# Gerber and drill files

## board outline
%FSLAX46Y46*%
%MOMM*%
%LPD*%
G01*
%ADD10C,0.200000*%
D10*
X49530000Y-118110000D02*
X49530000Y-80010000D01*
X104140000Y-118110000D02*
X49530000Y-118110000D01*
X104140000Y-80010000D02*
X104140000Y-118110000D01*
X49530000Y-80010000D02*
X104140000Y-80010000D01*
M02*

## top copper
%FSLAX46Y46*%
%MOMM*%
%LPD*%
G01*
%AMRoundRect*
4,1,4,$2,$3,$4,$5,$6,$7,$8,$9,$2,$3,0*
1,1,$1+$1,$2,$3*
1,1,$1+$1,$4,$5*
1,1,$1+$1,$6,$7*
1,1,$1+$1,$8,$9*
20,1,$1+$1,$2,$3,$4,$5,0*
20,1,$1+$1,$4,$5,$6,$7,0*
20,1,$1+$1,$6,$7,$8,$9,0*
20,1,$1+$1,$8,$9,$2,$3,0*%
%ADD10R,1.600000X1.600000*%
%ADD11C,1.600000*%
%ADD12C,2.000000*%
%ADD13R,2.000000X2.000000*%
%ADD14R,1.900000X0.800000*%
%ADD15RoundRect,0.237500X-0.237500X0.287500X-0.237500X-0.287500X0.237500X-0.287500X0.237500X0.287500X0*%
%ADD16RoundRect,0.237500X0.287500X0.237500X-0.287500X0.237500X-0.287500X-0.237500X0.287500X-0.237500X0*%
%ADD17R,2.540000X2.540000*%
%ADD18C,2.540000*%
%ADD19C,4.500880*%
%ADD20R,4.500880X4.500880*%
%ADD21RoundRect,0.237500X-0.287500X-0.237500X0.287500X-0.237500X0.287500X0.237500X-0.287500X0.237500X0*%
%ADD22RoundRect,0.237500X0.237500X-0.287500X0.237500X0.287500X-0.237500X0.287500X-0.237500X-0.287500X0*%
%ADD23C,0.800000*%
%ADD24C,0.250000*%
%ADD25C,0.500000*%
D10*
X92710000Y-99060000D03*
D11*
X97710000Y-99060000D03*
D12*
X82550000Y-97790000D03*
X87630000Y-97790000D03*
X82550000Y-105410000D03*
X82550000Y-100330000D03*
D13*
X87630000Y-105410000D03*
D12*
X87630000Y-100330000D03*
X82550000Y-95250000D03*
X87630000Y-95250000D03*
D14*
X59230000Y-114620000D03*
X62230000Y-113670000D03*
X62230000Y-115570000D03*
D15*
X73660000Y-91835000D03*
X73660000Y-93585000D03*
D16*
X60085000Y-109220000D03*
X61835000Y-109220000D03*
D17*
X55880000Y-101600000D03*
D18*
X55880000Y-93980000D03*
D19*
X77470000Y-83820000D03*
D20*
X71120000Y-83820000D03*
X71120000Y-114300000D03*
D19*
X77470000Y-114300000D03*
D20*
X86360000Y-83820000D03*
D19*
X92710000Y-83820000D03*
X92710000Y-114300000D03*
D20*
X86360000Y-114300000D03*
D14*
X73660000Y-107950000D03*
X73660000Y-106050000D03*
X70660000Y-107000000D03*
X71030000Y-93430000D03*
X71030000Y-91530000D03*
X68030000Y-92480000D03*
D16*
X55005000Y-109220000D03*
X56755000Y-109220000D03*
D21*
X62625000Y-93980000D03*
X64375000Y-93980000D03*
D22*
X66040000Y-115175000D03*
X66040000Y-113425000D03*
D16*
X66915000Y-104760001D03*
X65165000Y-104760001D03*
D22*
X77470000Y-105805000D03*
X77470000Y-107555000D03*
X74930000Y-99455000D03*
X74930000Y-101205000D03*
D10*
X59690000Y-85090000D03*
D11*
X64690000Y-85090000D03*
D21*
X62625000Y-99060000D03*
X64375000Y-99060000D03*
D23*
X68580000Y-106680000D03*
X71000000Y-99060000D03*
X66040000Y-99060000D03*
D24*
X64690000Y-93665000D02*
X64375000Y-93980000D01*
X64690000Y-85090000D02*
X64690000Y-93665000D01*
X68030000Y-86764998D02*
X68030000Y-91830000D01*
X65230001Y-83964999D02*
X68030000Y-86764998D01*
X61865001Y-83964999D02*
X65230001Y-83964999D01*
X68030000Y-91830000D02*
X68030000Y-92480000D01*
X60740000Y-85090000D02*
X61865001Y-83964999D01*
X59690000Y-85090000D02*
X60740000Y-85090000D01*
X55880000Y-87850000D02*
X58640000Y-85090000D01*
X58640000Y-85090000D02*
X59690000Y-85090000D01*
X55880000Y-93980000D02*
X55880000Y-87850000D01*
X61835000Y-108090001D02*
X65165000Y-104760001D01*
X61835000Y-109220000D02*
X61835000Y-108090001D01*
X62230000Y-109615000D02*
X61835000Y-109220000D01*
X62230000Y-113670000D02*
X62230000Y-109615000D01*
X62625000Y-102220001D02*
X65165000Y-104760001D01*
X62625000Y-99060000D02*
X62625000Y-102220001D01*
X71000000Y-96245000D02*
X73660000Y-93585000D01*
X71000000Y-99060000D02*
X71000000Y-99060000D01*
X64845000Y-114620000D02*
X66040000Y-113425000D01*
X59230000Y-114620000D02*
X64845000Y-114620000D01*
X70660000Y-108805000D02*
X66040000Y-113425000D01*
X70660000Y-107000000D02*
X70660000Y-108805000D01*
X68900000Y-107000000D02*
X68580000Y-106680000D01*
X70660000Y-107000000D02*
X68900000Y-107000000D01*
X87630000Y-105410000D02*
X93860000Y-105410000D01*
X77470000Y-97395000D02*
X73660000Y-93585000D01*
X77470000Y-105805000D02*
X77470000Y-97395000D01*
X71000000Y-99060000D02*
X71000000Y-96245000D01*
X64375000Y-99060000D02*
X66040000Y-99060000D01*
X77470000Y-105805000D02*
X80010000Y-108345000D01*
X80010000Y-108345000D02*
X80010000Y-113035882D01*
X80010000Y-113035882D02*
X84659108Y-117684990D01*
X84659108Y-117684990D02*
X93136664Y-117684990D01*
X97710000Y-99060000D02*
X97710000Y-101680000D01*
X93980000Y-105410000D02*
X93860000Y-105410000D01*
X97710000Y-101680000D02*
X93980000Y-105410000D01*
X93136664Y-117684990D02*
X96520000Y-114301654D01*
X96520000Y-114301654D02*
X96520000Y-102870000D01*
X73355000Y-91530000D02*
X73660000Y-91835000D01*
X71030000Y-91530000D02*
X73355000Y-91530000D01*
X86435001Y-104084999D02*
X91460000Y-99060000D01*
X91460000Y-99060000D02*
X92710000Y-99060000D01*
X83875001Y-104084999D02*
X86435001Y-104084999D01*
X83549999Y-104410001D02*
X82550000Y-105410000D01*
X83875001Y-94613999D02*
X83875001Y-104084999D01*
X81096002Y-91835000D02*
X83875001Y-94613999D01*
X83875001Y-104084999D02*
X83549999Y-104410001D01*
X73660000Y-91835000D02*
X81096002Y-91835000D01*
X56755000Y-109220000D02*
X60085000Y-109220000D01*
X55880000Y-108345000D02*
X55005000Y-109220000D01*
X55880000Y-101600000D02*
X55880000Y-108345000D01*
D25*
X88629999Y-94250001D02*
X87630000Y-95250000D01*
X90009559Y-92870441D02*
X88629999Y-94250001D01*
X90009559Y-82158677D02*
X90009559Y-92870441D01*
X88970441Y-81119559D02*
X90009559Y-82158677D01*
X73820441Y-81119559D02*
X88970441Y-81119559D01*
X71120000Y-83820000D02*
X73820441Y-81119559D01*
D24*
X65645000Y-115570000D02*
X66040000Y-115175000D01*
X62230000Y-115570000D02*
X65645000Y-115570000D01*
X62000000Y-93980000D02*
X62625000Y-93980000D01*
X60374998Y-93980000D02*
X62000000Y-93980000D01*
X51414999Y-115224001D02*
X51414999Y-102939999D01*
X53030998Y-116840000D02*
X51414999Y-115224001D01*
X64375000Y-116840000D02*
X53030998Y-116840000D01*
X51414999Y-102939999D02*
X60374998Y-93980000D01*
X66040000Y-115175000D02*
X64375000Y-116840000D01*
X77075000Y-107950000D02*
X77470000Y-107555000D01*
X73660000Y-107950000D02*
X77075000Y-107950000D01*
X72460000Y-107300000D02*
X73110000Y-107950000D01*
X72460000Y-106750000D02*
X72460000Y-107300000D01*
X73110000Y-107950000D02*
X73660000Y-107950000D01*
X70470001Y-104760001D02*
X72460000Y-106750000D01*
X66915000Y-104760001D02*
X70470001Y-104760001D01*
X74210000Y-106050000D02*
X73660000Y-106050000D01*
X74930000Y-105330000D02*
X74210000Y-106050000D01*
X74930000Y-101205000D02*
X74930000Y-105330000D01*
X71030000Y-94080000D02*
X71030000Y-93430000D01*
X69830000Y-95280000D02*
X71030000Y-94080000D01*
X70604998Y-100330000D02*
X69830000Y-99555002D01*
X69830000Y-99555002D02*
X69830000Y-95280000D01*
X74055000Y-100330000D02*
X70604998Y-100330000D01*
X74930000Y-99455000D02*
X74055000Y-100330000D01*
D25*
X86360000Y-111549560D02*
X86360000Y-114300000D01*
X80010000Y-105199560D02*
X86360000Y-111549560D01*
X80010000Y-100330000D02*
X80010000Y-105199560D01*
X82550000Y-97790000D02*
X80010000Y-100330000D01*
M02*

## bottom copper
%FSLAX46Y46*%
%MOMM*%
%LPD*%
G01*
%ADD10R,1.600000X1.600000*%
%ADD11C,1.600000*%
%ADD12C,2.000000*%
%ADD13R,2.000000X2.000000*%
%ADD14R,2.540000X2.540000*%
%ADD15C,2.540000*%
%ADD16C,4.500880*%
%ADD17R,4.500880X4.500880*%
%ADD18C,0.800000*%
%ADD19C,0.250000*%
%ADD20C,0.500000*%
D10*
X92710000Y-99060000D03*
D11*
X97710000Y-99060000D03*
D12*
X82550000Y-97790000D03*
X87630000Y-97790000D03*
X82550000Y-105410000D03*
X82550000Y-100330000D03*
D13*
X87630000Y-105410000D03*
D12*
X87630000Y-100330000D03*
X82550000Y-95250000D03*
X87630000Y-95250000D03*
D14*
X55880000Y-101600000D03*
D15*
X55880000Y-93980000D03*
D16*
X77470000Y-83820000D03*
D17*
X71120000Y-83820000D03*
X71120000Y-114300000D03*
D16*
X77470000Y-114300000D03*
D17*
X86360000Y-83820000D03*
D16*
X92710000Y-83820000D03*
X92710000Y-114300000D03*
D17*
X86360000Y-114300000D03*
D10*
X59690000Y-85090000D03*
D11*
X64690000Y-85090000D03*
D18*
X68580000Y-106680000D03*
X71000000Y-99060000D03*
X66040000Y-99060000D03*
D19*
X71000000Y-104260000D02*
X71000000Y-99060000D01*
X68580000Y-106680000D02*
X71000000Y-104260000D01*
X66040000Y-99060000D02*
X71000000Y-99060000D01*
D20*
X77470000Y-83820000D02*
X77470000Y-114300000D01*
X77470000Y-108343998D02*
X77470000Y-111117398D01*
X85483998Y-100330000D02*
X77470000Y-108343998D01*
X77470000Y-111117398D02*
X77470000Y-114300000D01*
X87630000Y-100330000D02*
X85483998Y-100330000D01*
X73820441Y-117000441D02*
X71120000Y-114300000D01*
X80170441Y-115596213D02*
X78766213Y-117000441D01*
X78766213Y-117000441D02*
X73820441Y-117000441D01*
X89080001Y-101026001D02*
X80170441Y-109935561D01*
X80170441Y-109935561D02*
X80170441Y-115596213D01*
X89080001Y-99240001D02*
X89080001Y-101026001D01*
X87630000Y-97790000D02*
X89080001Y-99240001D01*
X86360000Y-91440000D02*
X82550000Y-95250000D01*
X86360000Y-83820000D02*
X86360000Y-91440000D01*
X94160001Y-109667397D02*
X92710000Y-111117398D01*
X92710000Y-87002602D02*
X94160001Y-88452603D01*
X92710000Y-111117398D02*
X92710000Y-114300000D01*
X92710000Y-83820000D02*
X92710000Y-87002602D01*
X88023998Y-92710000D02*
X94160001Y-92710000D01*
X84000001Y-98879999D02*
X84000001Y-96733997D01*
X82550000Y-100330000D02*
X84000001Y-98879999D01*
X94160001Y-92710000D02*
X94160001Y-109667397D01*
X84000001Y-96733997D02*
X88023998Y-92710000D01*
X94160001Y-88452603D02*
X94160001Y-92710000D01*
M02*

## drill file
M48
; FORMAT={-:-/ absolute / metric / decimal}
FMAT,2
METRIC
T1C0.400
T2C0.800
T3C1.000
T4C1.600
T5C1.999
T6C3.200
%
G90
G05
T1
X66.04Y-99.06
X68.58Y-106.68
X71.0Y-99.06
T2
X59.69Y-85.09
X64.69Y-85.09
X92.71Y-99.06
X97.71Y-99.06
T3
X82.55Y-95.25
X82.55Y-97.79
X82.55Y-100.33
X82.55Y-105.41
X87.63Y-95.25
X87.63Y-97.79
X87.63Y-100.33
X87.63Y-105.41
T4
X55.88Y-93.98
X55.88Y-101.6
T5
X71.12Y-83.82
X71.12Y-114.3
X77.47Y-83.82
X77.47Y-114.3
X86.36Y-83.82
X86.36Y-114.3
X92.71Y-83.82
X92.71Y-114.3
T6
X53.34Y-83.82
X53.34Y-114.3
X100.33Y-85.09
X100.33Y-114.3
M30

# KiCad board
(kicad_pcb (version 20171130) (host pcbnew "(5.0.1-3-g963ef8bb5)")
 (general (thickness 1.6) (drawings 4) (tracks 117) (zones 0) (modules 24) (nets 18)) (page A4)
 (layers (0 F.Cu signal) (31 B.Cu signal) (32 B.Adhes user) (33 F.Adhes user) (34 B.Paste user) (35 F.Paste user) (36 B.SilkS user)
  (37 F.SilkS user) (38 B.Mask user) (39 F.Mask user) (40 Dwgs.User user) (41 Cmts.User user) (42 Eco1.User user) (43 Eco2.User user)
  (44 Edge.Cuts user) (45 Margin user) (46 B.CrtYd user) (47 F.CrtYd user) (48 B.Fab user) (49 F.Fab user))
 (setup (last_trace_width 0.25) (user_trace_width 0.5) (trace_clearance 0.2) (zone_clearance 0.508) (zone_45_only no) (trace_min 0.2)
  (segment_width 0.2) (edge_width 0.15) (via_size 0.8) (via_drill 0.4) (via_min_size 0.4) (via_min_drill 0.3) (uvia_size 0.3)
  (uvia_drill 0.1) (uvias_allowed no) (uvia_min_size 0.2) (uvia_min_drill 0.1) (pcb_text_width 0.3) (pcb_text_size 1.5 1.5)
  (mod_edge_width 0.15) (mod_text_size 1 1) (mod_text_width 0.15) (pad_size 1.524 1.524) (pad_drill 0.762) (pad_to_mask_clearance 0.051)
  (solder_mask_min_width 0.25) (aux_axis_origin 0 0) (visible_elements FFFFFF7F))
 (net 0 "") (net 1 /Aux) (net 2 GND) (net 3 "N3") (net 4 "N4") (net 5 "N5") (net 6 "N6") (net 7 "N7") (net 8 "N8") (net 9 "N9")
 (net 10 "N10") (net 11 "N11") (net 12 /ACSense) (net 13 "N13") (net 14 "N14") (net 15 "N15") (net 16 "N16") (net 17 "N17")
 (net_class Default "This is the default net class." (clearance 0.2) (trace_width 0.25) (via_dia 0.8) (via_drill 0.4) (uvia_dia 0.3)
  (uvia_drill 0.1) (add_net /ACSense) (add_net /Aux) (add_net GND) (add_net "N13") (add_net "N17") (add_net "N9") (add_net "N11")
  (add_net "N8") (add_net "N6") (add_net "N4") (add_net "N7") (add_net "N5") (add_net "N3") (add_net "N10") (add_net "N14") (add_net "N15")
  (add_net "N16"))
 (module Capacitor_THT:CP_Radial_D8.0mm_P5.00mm (layer F.Cu) (at 92.71 99.06)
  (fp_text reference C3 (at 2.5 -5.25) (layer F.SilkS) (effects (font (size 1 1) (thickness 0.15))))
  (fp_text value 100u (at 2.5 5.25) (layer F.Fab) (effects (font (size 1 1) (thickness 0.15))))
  (pad 1 thru_hole rect (at 0 0) (size 1.6 1.6) (drill 0.8) (layers *.Cu *.Mask) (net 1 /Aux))
  (pad 2 thru_hole circle (at 5 0) (size 1.6 1.6) (drill 0.8) (layers *.Cu *.Mask) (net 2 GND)))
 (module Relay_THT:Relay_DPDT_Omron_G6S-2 (layer F.Cu) (at 87.63 105.41 180)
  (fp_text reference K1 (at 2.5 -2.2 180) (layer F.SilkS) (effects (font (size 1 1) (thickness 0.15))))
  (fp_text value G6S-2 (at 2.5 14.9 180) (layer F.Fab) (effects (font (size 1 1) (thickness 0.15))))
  (pad 7 thru_hole circle (at 5.08 7.62 90) (size 2 2) (drill 1) (layers *.Cu *.Mask) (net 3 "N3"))
  (pad 4 thru_hole circle (at 0 7.62 90) (size 2 2) (drill 1) (layers *.Cu *.Mask) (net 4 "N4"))
  (pad 10 thru_hole circle (at 5.08 0 180) (size 2 2) (drill 1) (layers *.Cu *.Mask) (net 1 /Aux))
  (pad 8 thru_hole circle (at 5.08 5.08 180) (size 2 2) (drill 1) (layers *.Cu *.Mask) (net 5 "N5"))
  (pad 1 thru_hole rect (at 0 0 180) (size 2 2) (drill 1) (layers *.Cu *.Mask) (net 2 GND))
  (pad 3 thru_hole circle (at 0 5.08 180) (size 2 2) (drill 1) (layers *.Cu *.Mask) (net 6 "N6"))
  (pad 6 thru_hole circle (at 5.08 10.16 180) (size 2 2) (drill 1) (layers *.Cu *.Mask) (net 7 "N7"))
  (pad 5 thru_hole circle (at 0 10.16 180) (size 2 2) (drill 1) (layers *.Cu *.Mask) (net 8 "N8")))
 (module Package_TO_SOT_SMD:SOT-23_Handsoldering (layer F.Cu) (at 60.73 114.62 180)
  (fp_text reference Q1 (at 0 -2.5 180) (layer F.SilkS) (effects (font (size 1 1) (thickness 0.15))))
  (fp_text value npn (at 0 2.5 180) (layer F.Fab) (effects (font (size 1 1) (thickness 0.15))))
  (pad 3 smd rect (at 1.5 0 180) (size 1.9 0.8) (layers F.Cu F.Paste F.Mask) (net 2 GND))
  (pad 2 smd rect (at -1.5 0.95 180) (size 1.9 0.8) (layers F.Cu F.Paste F.Mask) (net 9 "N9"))
  (pad 1 smd rect (at -1.5 -0.95 180) (size 1.9 0.8) (layers F.Cu F.Paste F.Mask) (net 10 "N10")))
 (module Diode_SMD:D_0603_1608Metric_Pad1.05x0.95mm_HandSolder (layer F.Cu) (at 73.66 92.71 270)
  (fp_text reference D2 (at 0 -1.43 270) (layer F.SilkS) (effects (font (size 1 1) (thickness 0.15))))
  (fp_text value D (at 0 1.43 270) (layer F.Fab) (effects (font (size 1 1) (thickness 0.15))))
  (pad 1 smd roundrect (at -0.875 0 270) (size 1.05 0.95) (layers F.Cu F.Paste F.Mask) (roundrect_rratio 0.25) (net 1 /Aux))
  (pad 2 smd roundrect (at 0.875 0 270) (size 1.05 0.95) (layers F.Cu F.Paste F.Mask) (roundrect_rratio 0.25) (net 2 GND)))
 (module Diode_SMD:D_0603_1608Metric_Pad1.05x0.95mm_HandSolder (layer F.Cu) (at 60.96 109.22 180)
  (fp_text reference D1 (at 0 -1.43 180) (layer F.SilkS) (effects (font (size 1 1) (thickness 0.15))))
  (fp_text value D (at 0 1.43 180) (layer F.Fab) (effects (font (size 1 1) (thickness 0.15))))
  (pad 2 smd roundrect (at 0.875 0 180) (size 1.05 0.95) (layers F.Cu F.Paste F.Mask) (roundrect_rratio 0.25) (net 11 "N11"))
  (pad 1 smd roundrect (at -0.875 0 180) (size 1.05 0.95) (layers F.Cu F.Paste F.Mask) (roundrect_rratio 0.25) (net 9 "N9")))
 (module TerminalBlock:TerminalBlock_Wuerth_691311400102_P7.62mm (layer F.Cu) (at 55.88 101.6 90)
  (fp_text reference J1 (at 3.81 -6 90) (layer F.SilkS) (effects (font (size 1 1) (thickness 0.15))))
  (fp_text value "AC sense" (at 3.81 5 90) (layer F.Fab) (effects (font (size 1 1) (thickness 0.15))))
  (pad 1 thru_hole rect (at 0 0 90) (size 2.54 2.54) (drill 1.6) (layers *.Cu *.Mask) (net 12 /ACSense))
  (pad 2 thru_hole circle (at 7.62 0 90) (size 2.54 2.54) (drill 1.6) (layers *.Cu *.Mask) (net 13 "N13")))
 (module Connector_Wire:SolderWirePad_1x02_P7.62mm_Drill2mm (layer F.Cu) (at 71.12 83.82)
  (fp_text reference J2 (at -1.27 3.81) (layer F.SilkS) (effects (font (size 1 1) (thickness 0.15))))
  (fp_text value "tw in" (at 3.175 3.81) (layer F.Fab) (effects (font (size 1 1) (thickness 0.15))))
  (pad 2 thru_hole circle (at 6.35 0) (size 4.50088 4.50088) (drill 1.99898) (layers *.Cu *.Mask) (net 6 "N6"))
  (pad 1 thru_hole rect (at 0 0) (size 4.50088 4.50088) (drill 1.99898) (layers *.Cu *.Mask) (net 8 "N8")))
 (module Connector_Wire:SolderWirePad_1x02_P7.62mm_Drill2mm (layer F.Cu) (at 71.12 114.3)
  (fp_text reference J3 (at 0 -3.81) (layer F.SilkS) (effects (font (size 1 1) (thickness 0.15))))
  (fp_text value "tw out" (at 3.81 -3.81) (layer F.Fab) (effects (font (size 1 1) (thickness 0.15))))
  (pad 1 thru_hole rect (at 0 0) (size 4.50088 4.50088) (drill 1.99898) (layers *.Cu *.Mask) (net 4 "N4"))
  (pad 2 thru_hole circle (at 6.35 0) (size 4.50088 4.50088) (drill 1.99898) (layers *.Cu *.Mask) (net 6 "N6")))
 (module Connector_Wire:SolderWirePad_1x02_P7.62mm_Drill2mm (layer F.Cu) (at 86.36 83.82)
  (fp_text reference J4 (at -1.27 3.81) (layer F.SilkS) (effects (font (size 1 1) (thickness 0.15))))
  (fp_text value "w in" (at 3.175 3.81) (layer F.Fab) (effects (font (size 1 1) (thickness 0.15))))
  (pad 1 thru_hole rect (at 0 0) (size 4.50088 4.50088) (drill 1.99898) (layers *.Cu *.Mask) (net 7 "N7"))
  (pad 2 thru_hole circle (at 6.35 0) (size 4.50088 4.50088) (drill 1.99898) (layers *.Cu *.Mask) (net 5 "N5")))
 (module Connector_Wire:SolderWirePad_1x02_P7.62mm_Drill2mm (layer F.Cu) (at 86.36 114.3)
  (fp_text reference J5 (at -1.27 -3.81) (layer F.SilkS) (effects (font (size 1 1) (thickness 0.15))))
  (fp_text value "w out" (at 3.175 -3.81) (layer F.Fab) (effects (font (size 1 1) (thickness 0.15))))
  (pad 2 thru_hole circle (at 6.35 0) (size 4.50088 4.50088) (drill 1.99898) (layers *.Cu *.Mask) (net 5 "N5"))
  (pad 1 thru_hole rect (at 0 0) (size 4.50088 4.50088) (drill 1.99898) (layers *.Cu *.Mask) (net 3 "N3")))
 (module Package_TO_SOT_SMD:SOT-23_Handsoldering (layer F.Cu) (at 72.16 107 180)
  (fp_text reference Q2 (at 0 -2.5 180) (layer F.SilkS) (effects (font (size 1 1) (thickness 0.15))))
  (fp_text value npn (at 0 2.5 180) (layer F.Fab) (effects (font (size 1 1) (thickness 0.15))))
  (pad 1 smd rect (at -1.5 -0.95 180) (size 1.9 0.8) (layers F.Cu F.Paste F.Mask) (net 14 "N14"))
  (pad 2 smd rect (at -1.5 0.95 180) (size 1.9 0.8) (layers F.Cu F.Paste F.Mask) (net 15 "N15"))
  (pad 3 smd rect (at 1.5 0 180) (size 1.9 0.8) (layers F.Cu F.Paste F.Mask) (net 2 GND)))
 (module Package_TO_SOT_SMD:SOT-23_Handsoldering (layer F.Cu) (at 69.53 92.48 180)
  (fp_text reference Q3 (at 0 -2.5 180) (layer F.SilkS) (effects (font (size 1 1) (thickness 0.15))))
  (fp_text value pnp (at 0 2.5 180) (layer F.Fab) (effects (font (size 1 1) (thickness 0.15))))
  (pad 1 smd rect (at -1.5 -0.95 180) (size 1.9 0.8) (layers F.Cu F.Paste F.Mask) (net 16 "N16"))
  (pad 2 smd rect (at -1.5 0.95 180) (size 1.9 0.8) (layers F.Cu F.Paste F.Mask) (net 1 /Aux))
  (pad 3 smd rect (at 1.5 0 180) (size 1.9 0.8) (layers F.Cu F.Paste F.Mask) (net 13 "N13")))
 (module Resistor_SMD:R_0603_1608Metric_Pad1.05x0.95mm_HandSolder (layer F.Cu) (at 55.88 109.22 180)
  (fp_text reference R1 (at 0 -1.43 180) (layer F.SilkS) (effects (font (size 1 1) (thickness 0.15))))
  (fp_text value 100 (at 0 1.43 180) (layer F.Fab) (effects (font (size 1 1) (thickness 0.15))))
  (pad 2 smd roundrect (at 0.875 0 180) (size 1.05 0.95) (layers F.Cu F.Paste F.Mask) (roundrect_rratio 0.25) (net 12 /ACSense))
  (pad 1 smd roundrect (at -0.875 0 180) (size 1.05 0.95) (layers F.Cu F.Paste F.Mask) (roundrect_rratio 0.25) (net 11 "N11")))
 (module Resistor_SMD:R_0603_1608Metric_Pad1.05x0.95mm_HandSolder (layer F.Cu) (at 63.5 93.98)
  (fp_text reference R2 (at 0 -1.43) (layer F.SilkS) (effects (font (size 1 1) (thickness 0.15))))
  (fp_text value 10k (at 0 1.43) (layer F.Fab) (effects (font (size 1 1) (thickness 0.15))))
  (pad 1 smd roundrect (at -0.875 0) (size 1.05 0.95) (layers F.Cu F.Paste F.Mask) (roundrect_rratio 0.25) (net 10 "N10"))
  (pad 2 smd roundrect (at 0.875 0) (size 1.05 0.95) (layers F.Cu F.Paste F.Mask) (roundrect_rratio 0.25) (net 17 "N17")))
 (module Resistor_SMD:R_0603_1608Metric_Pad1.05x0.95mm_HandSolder (layer F.Cu) (at 66.04 114.3 90)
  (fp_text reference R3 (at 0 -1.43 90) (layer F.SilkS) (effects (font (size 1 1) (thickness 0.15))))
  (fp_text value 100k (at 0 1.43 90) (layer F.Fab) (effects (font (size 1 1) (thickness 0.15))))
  (pad 1 smd roundrect (at -0.875 0 90) (size 1.05 0.95) (layers F.Cu F.Paste F.Mask) (roundrect_rratio 0.25) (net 10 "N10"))
  (pad 2 smd roundrect (at 0.875 0 90) (size 1.05 0.95) (layers F.Cu F.Paste F.Mask) (roundrect_rratio 0.25) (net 2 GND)))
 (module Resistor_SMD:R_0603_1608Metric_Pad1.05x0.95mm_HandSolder (layer F.Cu) (at 66.04 104.760001 180)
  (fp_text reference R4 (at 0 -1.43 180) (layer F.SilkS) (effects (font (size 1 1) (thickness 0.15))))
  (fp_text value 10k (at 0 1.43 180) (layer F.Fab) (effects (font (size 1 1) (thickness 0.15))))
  (pad 1 smd roundrect (at -0.875 0 180) (size 1.05 0.95) (layers F.Cu F.Paste F.Mask) (roundrect_rratio 0.25) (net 14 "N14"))
  (pad 2 smd roundrect (at 0.875 0 180) (size 1.05 0.95) (layers F.Cu F.Paste F.Mask) (roundrect_rratio 0.25) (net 9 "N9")))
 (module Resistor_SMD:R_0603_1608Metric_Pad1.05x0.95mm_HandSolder (layer F.Cu) (at 77.47 106.68 90)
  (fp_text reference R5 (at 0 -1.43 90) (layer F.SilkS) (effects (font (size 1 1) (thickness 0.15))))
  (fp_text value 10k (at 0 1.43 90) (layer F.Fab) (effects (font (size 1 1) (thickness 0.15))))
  (pad 2 smd roundrect (at 0.875 0 90) (size 1.05 0.95) (layers F.Cu F.Paste F.Mask) (roundrect_rratio 0.25) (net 2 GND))
  (pad 1 smd roundrect (at -0.875 0 90) (size 1.05 0.95) (layers F.Cu F.Paste F.Mask) (roundrect_rratio 0.25) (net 14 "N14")))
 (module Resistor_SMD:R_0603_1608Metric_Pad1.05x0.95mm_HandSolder (layer F.Cu) (at 74.93 100.33 90)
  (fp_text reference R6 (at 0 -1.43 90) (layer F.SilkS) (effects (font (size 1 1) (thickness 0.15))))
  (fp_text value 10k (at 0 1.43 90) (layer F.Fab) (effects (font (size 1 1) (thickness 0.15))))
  (pad 2 smd roundrect (at 0.875 0 90) (size 1.05 0.95) (layers F.Cu F.Paste F.Mask) (roundrect_rratio 0.25) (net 16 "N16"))
  (pad 1 smd roundrect (at -0.875 0 90) (size 1.05 0.95) (layers F.Cu F.Paste F.Mask) (roundrect_rratio 0.25) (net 15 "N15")))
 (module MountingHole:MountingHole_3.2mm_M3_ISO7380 (layer F.Cu) (at 53.34 83.82)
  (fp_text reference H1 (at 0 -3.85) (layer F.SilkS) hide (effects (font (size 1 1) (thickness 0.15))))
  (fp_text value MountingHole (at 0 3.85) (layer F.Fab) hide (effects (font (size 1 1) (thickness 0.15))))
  (pad 1 np_thru_hole circle (at 0 0) (size 3.2 3.2) (drill 3.2) (layers *.Cu *.Mask)))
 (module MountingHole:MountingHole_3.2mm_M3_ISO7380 (layer F.Cu) (at 53.34 114.3)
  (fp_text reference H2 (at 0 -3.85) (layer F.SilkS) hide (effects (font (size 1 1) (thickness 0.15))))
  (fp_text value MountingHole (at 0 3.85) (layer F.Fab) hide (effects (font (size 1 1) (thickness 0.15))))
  (pad 1 np_thru_hole circle (at 0 0) (size 3.2 3.2) (drill 3.2) (layers *.Cu *.Mask)))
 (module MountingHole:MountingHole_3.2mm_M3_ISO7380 (layer F.Cu) (at 100.33 85.09)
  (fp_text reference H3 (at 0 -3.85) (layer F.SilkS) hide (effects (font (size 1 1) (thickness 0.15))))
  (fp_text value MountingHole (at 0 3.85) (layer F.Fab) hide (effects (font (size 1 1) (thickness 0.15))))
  (pad 1 np_thru_hole circle (at 0 0) (size 3.2 3.2) (drill 3.2) (layers *.Cu *.Mask)))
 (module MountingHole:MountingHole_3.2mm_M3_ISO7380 (layer F.Cu) (at 100.33 114.3)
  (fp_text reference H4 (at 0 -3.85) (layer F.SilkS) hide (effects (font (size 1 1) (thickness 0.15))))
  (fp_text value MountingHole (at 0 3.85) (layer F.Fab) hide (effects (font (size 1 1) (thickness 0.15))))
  (pad 1 np_thru_hole circle (at 0 0) (size 3.2 3.2) (drill 3.2) (layers *.Cu *.Mask)))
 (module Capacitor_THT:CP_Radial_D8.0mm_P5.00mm (layer F.Cu) (at 59.69 85.09)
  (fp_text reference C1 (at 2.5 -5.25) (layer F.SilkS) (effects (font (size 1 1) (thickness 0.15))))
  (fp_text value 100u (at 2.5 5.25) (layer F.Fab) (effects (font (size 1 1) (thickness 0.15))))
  (pad 1 thru_hole rect (at 0 0) (size 1.6 1.6) (drill 0.8) (layers *.Cu *.Mask) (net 13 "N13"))
  (pad 2 thru_hole circle (at 5 0) (size 1.6 1.6) (drill 0.8) (layers *.Cu *.Mask) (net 17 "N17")))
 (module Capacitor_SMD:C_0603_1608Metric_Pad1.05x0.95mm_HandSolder (layer F.Cu) (at 63.5 99.06)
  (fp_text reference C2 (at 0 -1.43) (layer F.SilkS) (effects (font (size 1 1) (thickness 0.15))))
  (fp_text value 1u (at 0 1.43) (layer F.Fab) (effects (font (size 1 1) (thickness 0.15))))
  (pad 1 smd roundrect (at -0.875 0) (size 1.05 0.95) (layers F.Cu F.Paste F.Mask) (roundrect_rratio 0.25) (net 9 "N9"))
  (pad 2 smd roundrect (at 0.875 0) (size 1.05 0.95) (layers F.Cu F.Paste F.Mask) (roundrect_rratio 0.25) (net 2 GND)))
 (gr_line (start 49.53 118.11) (end 49.53 80.01) (layer Edge.Cuts) (width 0.2))
 (gr_line (start 104.14 118.11) (end 49.53 118.11) (layer Edge.Cuts) (width 0.2))
 (gr_line (start 104.14 80.01) (end 104.14 118.11) (layer Edge.Cuts) (width 0.2))
 (gr_line (start 49.53 80.01) (end 104.14 80.01) (layer Edge.Cuts) (width 0.2))
 (segment (start 64.69 93.665) (end 64.375 93.98) (width 0.25) (layer F.Cu) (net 17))
 (segment (start 64.69 85.09) (end 64.69 93.665) (width 0.25) (layer F.Cu) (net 17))
 (segment (start 68.03 86.764998) (end 68.03 91.83) (width 0.25) (layer F.Cu) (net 13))
 (segment (start 65.230001 83.964999) (end 68.03 86.764998) (width 0.25) (layer F.Cu) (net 13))
 (segment (start 61.865001 83.964999) (end 65.230001 83.964999) (width 0.25) (layer F.Cu) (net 13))
 (segment (start 68.03 91.83) (end 68.03 92.48) (width 0.25) (layer F.Cu) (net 13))
 (segment (start 60.74 85.09) (end 61.865001 83.964999) (width 0.25) (layer F.Cu) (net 13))
 (segment (start 59.69 85.09) (end 60.74 85.09) (width 0.25) (layer F.Cu) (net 13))
 (segment (start 55.88 87.85) (end 58.64 85.09) (width 0.25) (layer F.Cu) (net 13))
 (segment (start 58.64 85.09) (end 59.69 85.09) (width 0.25) (layer F.Cu) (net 13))
 (segment (start 55.88 93.98) (end 55.88 87.85) (width 0.25) (layer F.Cu) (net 13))
 (segment (start 61.835 108.090001) (end 65.165 104.760001) (width 0.25) (layer F.Cu) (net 9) (status 20))
 (segment (start 61.835 109.22) (end 61.835 108.090001) (width 0.25) (layer F.Cu) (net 9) (status 10))
 (segment (start 62.23 109.615) (end 61.835 109.22) (width 0.25) (layer F.Cu) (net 9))
 (segment (start 62.23 113.67) (end 62.23 109.615) (width 0.25) (layer F.Cu) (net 9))
 (segment (start 62.625 102.220001) (end 65.165 104.760001) (width 0.25) (layer F.Cu) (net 9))
 (segment (start 62.625 99.06) (end 62.625 102.220001) (width 0.25) (layer F.Cu) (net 9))
 (segment (start 71 96.245) (end 73.66 93.585) (width 0.25) (layer F.Cu) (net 2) (status 20))
 (segment (start 71 99.06) (end 71 99.06) (width 0.25) (layer F.Cu) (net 2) (status 10))
 (segment (start 64.845 114.62) (end 66.04 113.425) (width 0.25) (layer F.Cu) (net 2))
 (segment (start 59.23 114.62) (end 64.845 114.62) (width 0.25) (layer F.Cu) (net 2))
 (segment (start 70.66 108.805) (end 66.04 113.425) (width 0.25) (layer F.Cu) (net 2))
 (segment (start 70.66 107) (end 70.66 108.805) (width 0.25) (layer F.Cu) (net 2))
 (via (at 68.58 106.68) (size 0.8) (drill 0.4) (layers F.Cu B.Cu) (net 2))
 (segment (start 68.9 107) (end 68.58 106.68) (width 0.25) (layer F.Cu) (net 2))
 (segment (start 70.66 107) (end 68.9 107) (width 0.25) (layer F.Cu) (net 2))
 (segment (start 71 104.26) (end 71 99.06) (width 0.25) (layer B.Cu) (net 2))
 (segment (start 68.58 106.68) (end 71 104.26) (width 0.25) (layer B.Cu) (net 2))
 (segment (start 87.63 105.41) (end 93.86 105.41) (width 0.25) (layer F.Cu) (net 2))
 (segment (start 77.47 97.395) (end 73.66 93.585) (width 0.25) (layer F.Cu) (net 2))
 (segment (start 77.47 105.805) (end 77.47 97.395) (width 0.25) (layer F.Cu) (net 2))
 (segment (start 71 99.06) (end 71 96.245) (width 0.25) (layer F.Cu) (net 2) (status 10))
 (via (at 71 99.06) (size 0.8) (drill 0.4) (layers F.Cu B.Cu) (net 2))
 (via (at 66.04 99.06) (size 0.8) (drill 0.4) (layers F.Cu B.Cu) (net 2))
 (segment (start 64.375 99.06) (end 66.04 99.06) (width 0.25) (layer F.Cu) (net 2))
 (segment (start 66.04 99.06) (end 71 99.06) (width 0.25) (layer B.Cu) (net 2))
 (segment (start 77.47 105.805) (end 80.01 108.345) (width 0.25) (layer F.Cu) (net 2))
 (segment (start 80.01 108.345) (end 80.01 113.035882) (width 0.25) (layer F.Cu) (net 2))
 (segment (start 80.01 113.035882) (end 84.659108 117.68499) (width 0.25) (layer F.Cu) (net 2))
 (segment (start 84.659108 117.68499) (end 93.136664 117.68499) (width 0.25) (layer F.Cu) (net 2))
 (segment (start 97.71 99.06) (end 97.71 101.68) (width 0.25) (layer F.Cu) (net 2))
 (segment (start 93.98 105.41) (end 93.86 105.41) (width 0.25) (layer F.Cu) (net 2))
 (segment (start 97.71 101.68) (end 93.98 105.41) (width 0.25) (layer F.Cu) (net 2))
 (segment (start 93.136664 117.68499) (end 96.52 114.301654) (width 0.25) (layer F.Cu) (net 2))
 (segment (start 96.52 114.301654) (end 96.52 102.87) (width 0.25) (layer F.Cu) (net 2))
 (segment (start 73.355 91.53) (end 73.66 91.835) (width 0.25) (layer F.Cu) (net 1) (status 30))
 (segment (start 71.03 91.53) (end 73.355 91.53) (width 0.25) (layer F.Cu) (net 1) (status 30))
 (segment (start 86.435001 104.084999) (end 91.46 99.06) (width 0.25) (layer F.Cu) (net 1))
 (segment (start 91.46 99.06) (end 92.71 99.06) (width 0.25) (layer F.Cu) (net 1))
 (segment (start 83.875001 104.084999) (end 86.435001 104.084999) (width 0.25) (layer F.Cu) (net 1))
 (segment (start 83.549999 104.410001) (end 82.55 105.41) (width 0.25) (layer F.Cu) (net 1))
 (segment (start 83.875001 94.613999) (end 83.875001 104.084999) (width 0.25) (layer F.Cu) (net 1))
 (segment (start 81.096002 91.835) (end 83.875001 94.613999) (width 0.25) (layer F.Cu) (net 1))
 (segment (start 83.875001 104.084999) (end 83.549999 104.410001) (width 0.25) (layer F.Cu) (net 1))
 (segment (start 73.66 91.835) (end 81.096002 91.835) (width 0.25) (layer F.Cu) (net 1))
 (segment (start 56.755 109.22) (end 60.085 109.22) (width 0.25) (layer F.Cu) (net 11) (status 30))
 (segment (start 55.88 108.345) (end 55.005 109.22) (width 0.25) (layer F.Cu) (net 12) (status 20))
 (segment (start 55.88 101.6) (end 55.88 108.345) (width 0.25) (layer F.Cu) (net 12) (status 10))
 (segment (start 77.47 83.82) (end 77.47 114.3) (width 0.5) (layer B.Cu) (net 6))
 (segment (start 77.47 108.343998) (end 77.47 111.117398) (width 0.5) (layer B.Cu) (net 6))
 (segment (start 85.483998 100.33) (end 77.47 108.343998) (width 0.5) (layer B.Cu) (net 6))
 (segment (start 77.47 111.117398) (end 77.47 114.3) (width 0.5) (layer B.Cu) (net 6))
 (segment (start 87.63 100.33) (end 85.483998 100.33) (width 0.5) (layer B.Cu) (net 6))
 (segment (start 88.629999 94.250001) (end 87.63 95.25) (width 0.5) (layer F.Cu) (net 8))
 (segment (start 90.009559 92.870441) (end 88.629999 94.250001) (width 0.5) (layer F.Cu) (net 8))
 (segment (start 90.009559 82.158677) (end 90.009559 92.870441) (width 0.5) (layer F.Cu) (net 8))
 (segment (start 88.970441 81.119559) (end 90.009559 82.158677) (width 0.5) (layer F.Cu) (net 8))
 (segment (start 73.820441 81.119559) (end 88.970441 81.119559) (width 0.5) (layer F.Cu) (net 8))
 (segment (start 71.12 83.82) (end 73.820441 81.119559) (width 0.5) (layer F.Cu) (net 8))
 (segment (start 73.820441 117.000441) (end 71.12 114.3) (width 0.5) (layer B.Cu) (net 4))
 (segment (start 80.170441 115.596213) (end 78.766213 117.000441) (width 0.5) (layer B.Cu) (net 4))
 (segment (start 78.766213 117.000441) (end 73.820441 117.000441) (width 0.5) (layer B.Cu) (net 4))
 (segment (start 89.080001 101.026001) (end 80.170441 109.935561) (width 0.5) (layer B.Cu) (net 4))
 (segment (start 80.170441 109.935561) (end 80.170441 115.596213) (width 0.5) (layer B.Cu) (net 4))
 (segment (start 89.080001 99.240001) (end 89.080001 101.026001) (width 0.5) (layer B.Cu) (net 4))
 (segment (start 87.63 97.79) (end 89.080001 99.240001) (width 0.5) (layer B.Cu) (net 4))
 (segment (start 86.36 91.44) (end 82.55 95.25) (width 0.5) (layer B.Cu) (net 7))
 (segment (start 86.36 83.82) (end 86.36 91.44) (width 0.5) (layer B.Cu) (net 7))
 (segment (start 94.160001 109.667397) (end 92.71 111.117398) (width 0.5) (layer B.Cu) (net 5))
 (segment (start 92.71 87.002602) (end 94.160001 88.452603) (width 0.5) (layer B.Cu) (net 5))
 (segment (start 92.71 111.117398) (end 92.71 114.3) (width 0.5) (layer B.Cu) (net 5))
 (segment (start 92.71 83.82) (end 92.71 87.002602) (width 0.5) (layer B.Cu) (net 5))
 (segment (start 88.023998 92.71) (end 94.160001 92.71) (width 0.5) (layer B.Cu) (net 5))
 (segment (start 84.000001 98.879999) (end 84.000001 96.733997) (width 0.5) (layer B.Cu) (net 5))
 (segment (start 82.55 100.33) (end 84.000001 98.879999) (width 0.5) (layer B.Cu) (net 5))
 (segment (start 94.160001 92.71) (end 94.160001 109.667397) (width 0.5) (layer B.Cu) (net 5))
 (segment (start 84.000001 96.733997) (end 88.023998 92.71) (width 0.5) (layer B.Cu) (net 5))
 (segment (start 94.160001 88.452603) (end 94.160001 92.71) (width 0.5) (layer B.Cu) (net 5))
 (segment (start 65.645 115.57) (end 66.04 115.175) (width 0.25) (layer F.Cu) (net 10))
 (segment (start 62.23 115.57) (end 65.645 115.57) (width 0.25) (layer F.Cu) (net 10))
 (segment (start 62 93.98) (end 62.625 93.98) (width 0.25) (layer F.Cu) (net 10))
 (segment (start 60.374998 93.98) (end 62 93.98) (width 0.25) (layer F.Cu) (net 10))
 (segment (start 51.414999 115.224001) (end 51.414999 102.939999) (width 0.25) (layer F.Cu) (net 10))
 (segment (start 53.030998 116.84) (end 51.414999 115.224001) (width 0.25) (layer F.Cu) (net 10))
 (segment (start 64.375 116.84) (end 53.030998 116.84) (width 0.25) (layer F.Cu) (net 10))
 (segment (start 51.414999 102.939999) (end 60.374998 93.98) (width 0.25) (layer F.Cu) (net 10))
 (segment (start 66.04 115.175) (end 64.375 116.84) (width 0.25) (layer F.Cu) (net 10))
 (segment (start 77.075 107.95) (end 77.47 107.555) (width 0.25) (layer F.Cu) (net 14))
 (segment (start 73.66 107.95) (end 77.075 107.95) (width 0.25) (layer F.Cu) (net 14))
 (segment (start 72.46 107.3) (end 73.11 107.95) (width 0.25) (layer F.Cu) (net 14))
 (segment (start 72.46 106.75) (end 72.46 107.3) (width 0.25) (layer F.Cu) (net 14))
 (segment (start 73.11 107.95) (end 73.66 107.95) (width 0.25) (layer F.Cu) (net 14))
 (segment (start 70.470001 104.760001) (end 72.46 106.75) (width 0.25) (layer F.Cu) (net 14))
 (segment (start 66.915 104.760001) (end 70.470001 104.760001) (width 0.25) (layer F.Cu) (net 14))
 (segment (start 74.21 106.05) (end 73.66 106.05) (width 0.25) (layer F.Cu) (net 15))
 (segment (start 74.93 105.33) (end 74.21 106.05) (width 0.25) (layer F.Cu) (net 15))
 (segment (start 74.93 101.205) (end 74.93 105.33) (width 0.25) (layer F.Cu) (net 15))
 (segment (start 71.03 94.08) (end 71.03 93.43) (width 0.25) (layer F.Cu) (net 16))
 (segment (start 69.83 95.28) (end 71.03 94.08) (width 0.25) (layer F.Cu) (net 16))
 (segment (start 70.604998 100.33) (end 69.83 99.555002) (width 0.25) (layer F.Cu) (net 16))
 (segment (start 69.83 99.555002) (end 69.83 95.28) (width 0.25) (layer F.Cu) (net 16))
 (segment (start 74.055 100.33) (end 70.604998 100.33) (width 0.25) (layer F.Cu) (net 16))
 (segment (start 74.93 99.455) (end 74.055 100.33) (width 0.25) (layer F.Cu) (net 16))
 (segment (start 86.36 111.54956) (end 86.36 114.3) (width 0.5) (layer F.Cu) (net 3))
 (segment (start 80.01 105.19956) (end 86.36 111.54956) (width 0.5) (layer F.Cu) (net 3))
 (segment (start 80.01 100.33) (end 80.01 105.19956) (width 0.5) (layer F.Cu) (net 3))
 (segment (start 82.55 97.79) (end 80.01 100.33) (width 0.5) (layer F.Cu) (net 3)))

